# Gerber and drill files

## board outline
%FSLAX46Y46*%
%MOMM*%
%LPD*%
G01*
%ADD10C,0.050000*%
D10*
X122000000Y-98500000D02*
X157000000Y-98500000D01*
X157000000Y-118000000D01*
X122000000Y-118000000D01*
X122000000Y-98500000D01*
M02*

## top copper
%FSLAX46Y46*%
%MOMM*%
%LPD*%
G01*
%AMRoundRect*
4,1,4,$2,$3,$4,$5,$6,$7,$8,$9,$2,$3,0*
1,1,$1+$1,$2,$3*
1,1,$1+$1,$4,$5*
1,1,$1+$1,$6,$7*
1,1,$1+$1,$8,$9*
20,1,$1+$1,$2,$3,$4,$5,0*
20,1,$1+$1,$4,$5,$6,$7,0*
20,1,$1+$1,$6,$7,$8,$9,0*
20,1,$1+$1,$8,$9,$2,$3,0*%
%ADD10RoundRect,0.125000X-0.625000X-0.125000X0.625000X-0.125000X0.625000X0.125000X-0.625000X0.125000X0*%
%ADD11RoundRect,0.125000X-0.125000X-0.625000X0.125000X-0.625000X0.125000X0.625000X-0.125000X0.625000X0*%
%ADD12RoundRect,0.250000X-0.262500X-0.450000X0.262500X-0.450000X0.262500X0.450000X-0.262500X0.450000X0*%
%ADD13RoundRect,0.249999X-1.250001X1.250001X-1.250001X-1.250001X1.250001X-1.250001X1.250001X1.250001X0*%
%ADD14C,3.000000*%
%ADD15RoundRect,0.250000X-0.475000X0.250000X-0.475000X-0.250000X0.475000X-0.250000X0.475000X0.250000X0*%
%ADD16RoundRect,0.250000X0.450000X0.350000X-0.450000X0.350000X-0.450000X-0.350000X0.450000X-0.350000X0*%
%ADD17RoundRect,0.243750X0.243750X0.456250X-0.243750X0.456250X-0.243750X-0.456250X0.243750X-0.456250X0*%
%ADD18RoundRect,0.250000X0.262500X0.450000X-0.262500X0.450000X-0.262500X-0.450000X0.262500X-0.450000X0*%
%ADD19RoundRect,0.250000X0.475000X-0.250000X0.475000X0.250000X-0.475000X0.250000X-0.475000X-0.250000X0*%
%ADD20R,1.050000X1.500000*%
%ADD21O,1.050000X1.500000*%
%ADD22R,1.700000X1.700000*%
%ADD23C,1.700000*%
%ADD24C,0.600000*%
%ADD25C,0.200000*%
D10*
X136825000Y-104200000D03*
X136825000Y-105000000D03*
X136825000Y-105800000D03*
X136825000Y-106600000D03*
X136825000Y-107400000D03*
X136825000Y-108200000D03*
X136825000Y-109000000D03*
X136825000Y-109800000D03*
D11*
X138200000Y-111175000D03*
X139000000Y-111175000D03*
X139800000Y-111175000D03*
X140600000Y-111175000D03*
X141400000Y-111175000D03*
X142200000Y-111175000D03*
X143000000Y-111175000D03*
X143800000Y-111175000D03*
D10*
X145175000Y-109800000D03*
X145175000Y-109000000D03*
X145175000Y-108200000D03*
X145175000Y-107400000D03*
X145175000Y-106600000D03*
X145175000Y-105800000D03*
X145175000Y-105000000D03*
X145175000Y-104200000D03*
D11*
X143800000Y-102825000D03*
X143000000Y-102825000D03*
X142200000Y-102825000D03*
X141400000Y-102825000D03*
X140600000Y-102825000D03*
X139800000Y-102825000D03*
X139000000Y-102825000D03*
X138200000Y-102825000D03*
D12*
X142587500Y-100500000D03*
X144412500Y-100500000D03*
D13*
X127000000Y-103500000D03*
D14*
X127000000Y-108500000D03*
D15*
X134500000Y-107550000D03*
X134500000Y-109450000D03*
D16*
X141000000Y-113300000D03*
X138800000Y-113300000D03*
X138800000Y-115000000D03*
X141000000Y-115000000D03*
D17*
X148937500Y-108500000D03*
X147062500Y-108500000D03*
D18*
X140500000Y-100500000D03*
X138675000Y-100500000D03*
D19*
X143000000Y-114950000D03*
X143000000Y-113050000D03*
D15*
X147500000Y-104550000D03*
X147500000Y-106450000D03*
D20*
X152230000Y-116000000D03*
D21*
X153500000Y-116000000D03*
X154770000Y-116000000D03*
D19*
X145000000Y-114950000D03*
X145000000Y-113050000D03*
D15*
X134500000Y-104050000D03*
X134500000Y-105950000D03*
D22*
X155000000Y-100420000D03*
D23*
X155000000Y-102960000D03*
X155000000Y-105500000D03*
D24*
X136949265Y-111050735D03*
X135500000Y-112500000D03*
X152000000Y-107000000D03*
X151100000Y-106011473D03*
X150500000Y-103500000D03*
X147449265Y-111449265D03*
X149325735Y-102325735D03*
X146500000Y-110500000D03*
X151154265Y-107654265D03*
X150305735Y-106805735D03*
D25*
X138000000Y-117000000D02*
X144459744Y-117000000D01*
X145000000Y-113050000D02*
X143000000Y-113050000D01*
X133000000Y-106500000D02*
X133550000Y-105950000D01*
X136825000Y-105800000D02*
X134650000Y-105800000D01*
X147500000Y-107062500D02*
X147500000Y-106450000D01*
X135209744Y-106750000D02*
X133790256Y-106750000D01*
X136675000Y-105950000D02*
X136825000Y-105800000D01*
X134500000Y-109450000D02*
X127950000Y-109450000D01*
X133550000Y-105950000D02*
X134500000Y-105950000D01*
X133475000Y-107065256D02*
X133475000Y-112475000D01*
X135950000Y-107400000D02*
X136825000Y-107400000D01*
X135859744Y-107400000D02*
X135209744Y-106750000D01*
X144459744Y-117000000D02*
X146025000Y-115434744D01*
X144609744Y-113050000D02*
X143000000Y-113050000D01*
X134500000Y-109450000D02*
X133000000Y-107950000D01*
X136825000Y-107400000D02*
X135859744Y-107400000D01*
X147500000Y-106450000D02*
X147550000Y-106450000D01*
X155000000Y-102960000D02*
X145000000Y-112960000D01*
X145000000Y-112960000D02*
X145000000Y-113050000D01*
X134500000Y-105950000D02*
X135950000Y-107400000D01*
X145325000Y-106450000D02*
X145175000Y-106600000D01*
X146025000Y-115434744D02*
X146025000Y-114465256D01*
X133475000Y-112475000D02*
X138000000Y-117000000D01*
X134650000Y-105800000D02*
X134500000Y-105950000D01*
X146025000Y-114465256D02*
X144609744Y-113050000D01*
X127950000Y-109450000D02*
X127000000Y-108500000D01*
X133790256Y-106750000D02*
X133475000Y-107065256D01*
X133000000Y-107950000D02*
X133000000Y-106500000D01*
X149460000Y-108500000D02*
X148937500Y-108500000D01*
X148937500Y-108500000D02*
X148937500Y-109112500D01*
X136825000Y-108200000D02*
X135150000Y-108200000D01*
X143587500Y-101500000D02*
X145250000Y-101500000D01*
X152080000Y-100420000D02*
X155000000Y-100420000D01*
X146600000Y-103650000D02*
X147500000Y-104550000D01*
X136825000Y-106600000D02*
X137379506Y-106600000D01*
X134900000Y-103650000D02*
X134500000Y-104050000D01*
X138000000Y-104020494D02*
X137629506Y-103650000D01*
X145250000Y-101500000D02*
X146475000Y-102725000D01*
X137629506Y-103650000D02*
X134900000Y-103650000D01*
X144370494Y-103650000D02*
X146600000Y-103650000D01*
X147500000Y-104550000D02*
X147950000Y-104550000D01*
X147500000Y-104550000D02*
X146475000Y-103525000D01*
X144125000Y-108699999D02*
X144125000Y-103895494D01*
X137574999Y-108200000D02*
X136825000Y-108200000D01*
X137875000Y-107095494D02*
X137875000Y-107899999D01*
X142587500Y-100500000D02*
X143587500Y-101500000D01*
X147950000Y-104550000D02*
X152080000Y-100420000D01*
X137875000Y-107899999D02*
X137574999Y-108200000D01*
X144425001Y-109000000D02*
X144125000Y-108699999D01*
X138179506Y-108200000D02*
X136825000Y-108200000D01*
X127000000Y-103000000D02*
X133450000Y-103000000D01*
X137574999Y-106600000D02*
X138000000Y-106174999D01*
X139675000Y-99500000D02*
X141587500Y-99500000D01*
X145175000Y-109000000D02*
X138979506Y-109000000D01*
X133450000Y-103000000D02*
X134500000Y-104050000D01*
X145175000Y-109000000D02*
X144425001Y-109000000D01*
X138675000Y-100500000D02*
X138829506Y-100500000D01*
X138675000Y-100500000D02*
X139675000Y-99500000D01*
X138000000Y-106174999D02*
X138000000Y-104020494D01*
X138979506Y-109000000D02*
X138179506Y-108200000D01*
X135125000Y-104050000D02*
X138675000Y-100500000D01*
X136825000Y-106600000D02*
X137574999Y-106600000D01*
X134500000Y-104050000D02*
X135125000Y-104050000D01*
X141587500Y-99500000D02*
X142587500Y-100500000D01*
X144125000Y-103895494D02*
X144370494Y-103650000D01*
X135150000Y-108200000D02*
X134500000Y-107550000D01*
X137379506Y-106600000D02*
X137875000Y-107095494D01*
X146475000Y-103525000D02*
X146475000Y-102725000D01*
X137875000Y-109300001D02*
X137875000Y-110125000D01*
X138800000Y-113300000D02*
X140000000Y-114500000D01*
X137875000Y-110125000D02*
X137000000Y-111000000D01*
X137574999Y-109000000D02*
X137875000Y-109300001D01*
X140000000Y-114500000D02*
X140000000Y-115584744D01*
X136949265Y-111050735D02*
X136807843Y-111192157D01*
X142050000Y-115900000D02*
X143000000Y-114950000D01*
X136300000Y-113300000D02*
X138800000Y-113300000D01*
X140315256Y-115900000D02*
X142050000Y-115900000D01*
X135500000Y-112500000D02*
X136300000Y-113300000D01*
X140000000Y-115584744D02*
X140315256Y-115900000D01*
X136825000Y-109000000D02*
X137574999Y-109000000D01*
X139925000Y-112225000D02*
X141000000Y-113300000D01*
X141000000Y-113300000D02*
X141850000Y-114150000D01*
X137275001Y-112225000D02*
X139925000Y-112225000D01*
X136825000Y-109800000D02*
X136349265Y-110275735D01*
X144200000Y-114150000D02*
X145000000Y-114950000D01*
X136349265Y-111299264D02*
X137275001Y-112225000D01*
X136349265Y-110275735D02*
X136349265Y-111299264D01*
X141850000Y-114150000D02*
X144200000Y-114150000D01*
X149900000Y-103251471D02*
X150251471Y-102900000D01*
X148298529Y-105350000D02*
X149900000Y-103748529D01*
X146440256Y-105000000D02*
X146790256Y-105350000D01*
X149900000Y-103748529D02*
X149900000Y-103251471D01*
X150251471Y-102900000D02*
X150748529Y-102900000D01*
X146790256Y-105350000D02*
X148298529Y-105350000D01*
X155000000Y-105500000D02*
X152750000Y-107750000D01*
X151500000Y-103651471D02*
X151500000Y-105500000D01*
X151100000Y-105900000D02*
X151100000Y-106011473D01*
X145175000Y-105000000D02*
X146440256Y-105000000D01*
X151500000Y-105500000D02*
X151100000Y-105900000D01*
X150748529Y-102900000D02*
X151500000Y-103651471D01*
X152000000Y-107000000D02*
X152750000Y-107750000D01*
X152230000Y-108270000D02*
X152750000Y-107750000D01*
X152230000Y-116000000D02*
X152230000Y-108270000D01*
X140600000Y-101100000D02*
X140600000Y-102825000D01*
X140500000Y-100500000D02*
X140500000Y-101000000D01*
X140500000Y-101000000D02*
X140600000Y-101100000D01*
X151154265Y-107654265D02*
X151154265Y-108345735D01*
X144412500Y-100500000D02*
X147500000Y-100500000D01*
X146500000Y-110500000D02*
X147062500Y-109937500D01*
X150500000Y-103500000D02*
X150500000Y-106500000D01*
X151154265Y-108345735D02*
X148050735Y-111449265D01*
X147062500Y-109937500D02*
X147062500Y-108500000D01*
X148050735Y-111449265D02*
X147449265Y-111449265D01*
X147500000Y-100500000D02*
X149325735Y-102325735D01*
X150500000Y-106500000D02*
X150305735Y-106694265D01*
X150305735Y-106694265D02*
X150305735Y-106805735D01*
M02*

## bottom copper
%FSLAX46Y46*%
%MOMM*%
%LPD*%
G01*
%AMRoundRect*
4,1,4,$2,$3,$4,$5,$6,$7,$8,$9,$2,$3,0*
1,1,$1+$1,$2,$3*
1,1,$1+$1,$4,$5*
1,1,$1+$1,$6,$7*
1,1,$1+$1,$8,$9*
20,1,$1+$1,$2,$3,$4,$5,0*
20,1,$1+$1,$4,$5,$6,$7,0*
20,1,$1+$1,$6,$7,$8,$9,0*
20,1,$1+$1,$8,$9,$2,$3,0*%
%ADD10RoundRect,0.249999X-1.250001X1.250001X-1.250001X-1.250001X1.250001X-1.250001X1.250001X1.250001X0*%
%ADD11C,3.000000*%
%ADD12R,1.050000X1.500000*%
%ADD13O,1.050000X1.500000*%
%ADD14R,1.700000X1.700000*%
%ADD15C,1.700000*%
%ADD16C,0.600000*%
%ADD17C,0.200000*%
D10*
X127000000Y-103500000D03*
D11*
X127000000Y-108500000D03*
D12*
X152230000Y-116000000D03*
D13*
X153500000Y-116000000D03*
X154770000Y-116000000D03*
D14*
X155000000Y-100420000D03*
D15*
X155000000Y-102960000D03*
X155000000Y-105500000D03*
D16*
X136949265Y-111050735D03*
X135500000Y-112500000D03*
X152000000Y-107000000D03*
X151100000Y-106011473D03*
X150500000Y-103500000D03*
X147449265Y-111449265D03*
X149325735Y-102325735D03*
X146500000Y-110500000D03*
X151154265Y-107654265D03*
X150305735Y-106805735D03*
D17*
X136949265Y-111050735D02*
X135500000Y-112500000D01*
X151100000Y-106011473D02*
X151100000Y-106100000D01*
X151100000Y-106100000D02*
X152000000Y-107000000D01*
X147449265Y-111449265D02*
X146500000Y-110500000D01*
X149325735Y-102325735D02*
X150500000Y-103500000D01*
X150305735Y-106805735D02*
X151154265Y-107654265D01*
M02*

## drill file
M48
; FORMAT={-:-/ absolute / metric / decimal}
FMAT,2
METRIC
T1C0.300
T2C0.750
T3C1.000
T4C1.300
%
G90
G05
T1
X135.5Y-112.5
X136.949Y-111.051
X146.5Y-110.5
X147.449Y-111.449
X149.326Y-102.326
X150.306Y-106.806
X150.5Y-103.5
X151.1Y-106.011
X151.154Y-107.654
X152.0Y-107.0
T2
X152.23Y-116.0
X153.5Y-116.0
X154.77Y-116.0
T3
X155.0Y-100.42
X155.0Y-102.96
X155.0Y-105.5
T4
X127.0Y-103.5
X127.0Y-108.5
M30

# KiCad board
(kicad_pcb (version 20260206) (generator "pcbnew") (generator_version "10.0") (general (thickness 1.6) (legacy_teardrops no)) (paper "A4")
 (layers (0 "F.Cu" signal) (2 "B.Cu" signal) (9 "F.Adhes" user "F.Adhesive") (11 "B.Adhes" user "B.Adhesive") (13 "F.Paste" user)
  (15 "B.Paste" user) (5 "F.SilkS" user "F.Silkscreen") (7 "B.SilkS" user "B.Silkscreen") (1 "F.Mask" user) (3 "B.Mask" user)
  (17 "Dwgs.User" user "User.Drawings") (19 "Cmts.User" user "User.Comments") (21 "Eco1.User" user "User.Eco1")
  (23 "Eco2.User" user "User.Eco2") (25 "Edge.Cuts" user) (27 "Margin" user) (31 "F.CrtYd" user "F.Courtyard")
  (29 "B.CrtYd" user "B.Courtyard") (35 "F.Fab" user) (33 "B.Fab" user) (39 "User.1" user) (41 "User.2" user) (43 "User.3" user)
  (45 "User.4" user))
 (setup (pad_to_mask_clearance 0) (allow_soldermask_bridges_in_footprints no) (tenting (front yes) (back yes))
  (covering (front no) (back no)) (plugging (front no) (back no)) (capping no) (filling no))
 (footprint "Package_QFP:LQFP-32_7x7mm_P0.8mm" (layer "F.Cu") (at 141 107)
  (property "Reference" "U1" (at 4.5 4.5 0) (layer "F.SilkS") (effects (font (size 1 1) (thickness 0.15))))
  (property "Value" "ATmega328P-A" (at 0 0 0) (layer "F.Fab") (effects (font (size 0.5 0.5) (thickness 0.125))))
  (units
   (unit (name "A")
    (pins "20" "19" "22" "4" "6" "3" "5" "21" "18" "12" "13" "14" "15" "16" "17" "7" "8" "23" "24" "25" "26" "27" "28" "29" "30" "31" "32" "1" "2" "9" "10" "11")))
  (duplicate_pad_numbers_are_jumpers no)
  (pad "1" smd roundrect (at -4.175 -2.8) (size 1.5 0.5) (layers "F.Cu" "F.Mask" "F.Paste") (roundrect_rratio 0.25)
   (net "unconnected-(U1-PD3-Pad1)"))
  (pad "2" smd roundrect (at -4.175 -2) (size 1.5 0.5) (layers "F.Cu" "F.Mask" "F.Paste") (roundrect_rratio 0.25)
   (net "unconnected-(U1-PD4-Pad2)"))
  (pad "3" smd roundrect (at -4.175 -1.2) (size 1.5 0.5) (layers "F.Cu" "F.Mask" "F.Paste") (roundrect_rratio 0.25) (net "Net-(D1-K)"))
  (pad "4" smd roundrect (at -4.175 -0.4) (size 1.5 0.5) (layers "F.Cu" "F.Mask" "F.Paste") (roundrect_rratio 0.25) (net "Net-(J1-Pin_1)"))
  (pad "5" smd roundrect (at -4.175 0.4) (size 1.5 0.5) (layers "F.Cu" "F.Mask" "F.Paste") (roundrect_rratio 0.25) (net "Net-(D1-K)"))
  (pad "6" smd roundrect (at -4.175 1.2) (size 1.5 0.5) (layers "F.Cu" "F.Mask" "F.Paste") (roundrect_rratio 0.25) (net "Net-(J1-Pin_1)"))
  (pad "7" smd roundrect (at -4.175 2) (size 1.5 0.5) (layers "F.Cu" "F.Mask" "F.Paste") (roundrect_rratio 0.25)
   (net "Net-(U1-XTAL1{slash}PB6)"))
  (pad "8" smd roundrect (at -4.175 2.8) (size 1.5 0.5) (layers "F.Cu" "F.Mask" "F.Paste") (roundrect_rratio 0.25)
   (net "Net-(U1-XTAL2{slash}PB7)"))
  (pad "9" smd roundrect (at -2.8 4.175) (size 0.5 1.5) (layers "F.Cu" "F.Mask" "F.Paste") (roundrect_rratio 0.25)
   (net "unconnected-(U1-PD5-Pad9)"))
  (pad "10" smd roundrect (at -2 4.175) (size 0.5 1.5) (layers "F.Cu" "F.Mask" "F.Paste") (roundrect_rratio 0.25)
   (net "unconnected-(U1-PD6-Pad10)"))
  (pad "11" smd roundrect (at -1.2 4.175) (size 0.5 1.5) (layers "F.Cu" "F.Mask" "F.Paste") (roundrect_rratio 0.25)
   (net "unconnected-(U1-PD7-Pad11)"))
  (pad "12" smd roundrect (at -0.4 4.175) (size 0.5 1.5) (layers "F.Cu" "F.Mask" "F.Paste") (roundrect_rratio 0.25)
   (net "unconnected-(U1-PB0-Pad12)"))
  (pad "13" smd roundrect (at 0.4 4.175) (size 0.5 1.5) (layers "F.Cu" "F.Mask" "F.Paste") (roundrect_rratio 0.25)
   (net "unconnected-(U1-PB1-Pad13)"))
  (pad "14" smd roundrect (at 1.2 4.175) (size 0.5 1.5) (layers "F.Cu" "F.Mask" "F.Paste") (roundrect_rratio 0.25)
   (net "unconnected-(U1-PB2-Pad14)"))
  (pad "15" smd roundrect (at 2 4.175) (size 0.5 1.5) (layers "F.Cu" "F.Mask" "F.Paste") (roundrect_rratio 0.25)
   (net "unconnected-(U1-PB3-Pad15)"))
  (pad "16" smd roundrect (at 2.8 4.175) (size 0.5 1.5) (layers "F.Cu" "F.Mask" "F.Paste") (roundrect_rratio 0.25)
   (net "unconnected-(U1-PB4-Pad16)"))
  (pad "17" smd roundrect (at 4.175 2.8) (size 1.5 0.5) (layers "F.Cu" "F.Mask" "F.Paste") (roundrect_rratio 0.25)
   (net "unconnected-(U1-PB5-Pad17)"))
  (pad "18" smd roundrect (at 4.175 2) (size 1.5 0.5) (layers "F.Cu" "F.Mask" "F.Paste") (roundrect_rratio 0.25) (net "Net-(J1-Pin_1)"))
  (pad "19" smd roundrect (at 4.175 1.2) (size 1.5 0.5) (layers "F.Cu" "F.Mask" "F.Paste") (roundrect_rratio 0.25)
   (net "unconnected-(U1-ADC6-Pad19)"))
  (pad "20" smd roundrect (at 4.175 0.4) (size 1.5 0.5) (layers "F.Cu" "F.Mask" "F.Paste") (roundrect_rratio 0.25)
   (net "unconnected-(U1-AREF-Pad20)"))
  (pad "21" smd roundrect (at 4.175 -0.4) (size 1.5 0.5) (layers "F.Cu" "F.Mask" "F.Paste") (roundrect_rratio 0.25) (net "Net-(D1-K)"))
  (pad "22" smd roundrect (at 4.175 -1.2) (size 1.5 0.5) (layers "F.Cu" "F.Mask" "F.Paste") (roundrect_rratio 0.25)
   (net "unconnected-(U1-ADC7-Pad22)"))
  (pad "23" smd roundrect (at 4.175 -2) (size 1.5 0.5) (layers "F.Cu" "F.Mask" "F.Paste") (roundrect_rratio 0.25) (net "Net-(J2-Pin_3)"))
  (pad "24" smd roundrect (at 4.175 -2.8) (size 1.5 0.5) (layers "F.Cu" "F.Mask" "F.Paste") (roundrect_rratio 0.25)
   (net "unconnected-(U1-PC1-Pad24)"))
  (pad "25" smd roundrect (at 2.8 -4.175) (size 0.5 1.5) (layers "F.Cu" "F.Mask" "F.Paste") (roundrect_rratio 0.25)
   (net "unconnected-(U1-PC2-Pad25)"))
  (pad "26" smd roundrect (at 2 -4.175) (size 0.5 1.5) (layers "F.Cu" "F.Mask" "F.Paste") (roundrect_rratio 0.25)
   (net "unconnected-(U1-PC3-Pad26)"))
  (pad "27" smd roundrect (at 1.2 -4.175) (size 0.5 1.5) (layers "F.Cu" "F.Mask" "F.Paste") (roundrect_rratio 0.25)
   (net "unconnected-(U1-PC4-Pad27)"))
  (pad "28" smd roundrect (at 0.4 -4.175) (size 0.5 1.5) (layers "F.Cu" "F.Mask" "F.Paste") (roundrect_rratio 0.25)
   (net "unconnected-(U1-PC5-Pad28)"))
  (pad "29" smd roundrect (at -0.4 -4.175) (size 0.5 1.5) (layers "F.Cu" "F.Mask" "F.Paste") (roundrect_rratio 0.25)
   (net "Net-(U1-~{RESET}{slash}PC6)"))
  (pad "30" smd roundrect (at -1.2 -4.175) (size 0.5 1.5) (layers "F.Cu" "F.Mask" "F.Paste") (roundrect_rratio 0.25)
   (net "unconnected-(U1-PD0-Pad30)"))
  (pad "31" smd roundrect (at -2 -4.175) (size 0.5 1.5) (layers "F.Cu" "F.Mask" "F.Paste") (roundrect_rratio 0.25)
   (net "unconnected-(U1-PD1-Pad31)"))
  (pad "32" smd roundrect (at -2.8 -4.175) (size 0.5 1.5) (layers "F.Cu" "F.Mask" "F.Paste") (roundrect_rratio 0.25)
   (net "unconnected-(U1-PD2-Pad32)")))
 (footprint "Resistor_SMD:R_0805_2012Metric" (layer "F.Cu") (at 143.5 100.5)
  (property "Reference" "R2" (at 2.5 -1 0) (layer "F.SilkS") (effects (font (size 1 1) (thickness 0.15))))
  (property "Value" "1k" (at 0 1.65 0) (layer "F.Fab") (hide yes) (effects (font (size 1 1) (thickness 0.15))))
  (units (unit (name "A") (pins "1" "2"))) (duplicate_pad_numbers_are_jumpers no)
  (pad "1" smd roundrect (at -0.9125 0) (size 1.025 1.4) (layers "F.Cu" "F.Mask" "F.Paste") (roundrect_rratio 0.243902)
   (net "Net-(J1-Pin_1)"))
  (pad "2" smd roundrect (at 0.9125 0) (size 1.025 1.4) (layers "F.Cu" "F.Mask" "F.Paste") (roundrect_rratio 0.243902) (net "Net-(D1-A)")))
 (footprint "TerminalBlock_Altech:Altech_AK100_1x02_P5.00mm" (layer "F.Cu") (at 127 103.5 -90)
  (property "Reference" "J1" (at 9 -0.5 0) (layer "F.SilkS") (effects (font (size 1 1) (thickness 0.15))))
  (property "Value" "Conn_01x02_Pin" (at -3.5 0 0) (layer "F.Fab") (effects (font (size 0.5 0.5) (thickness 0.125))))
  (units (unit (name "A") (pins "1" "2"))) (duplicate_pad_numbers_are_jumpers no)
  (pad "1" thru_hole roundrect (at 0 0 270) (size 3 3) (drill 1.3) (layers "*.Cu" "*.Mask") (remove_unused_layers no)
   (roundrect_rratio 0.083333) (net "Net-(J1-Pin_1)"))
  (pad "2" thru_hole circle (at 5 0 270) (size 3 3) (drill 1.3) (layers "*.Cu" "*.Mask") (remove_unused_layers no) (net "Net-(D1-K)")))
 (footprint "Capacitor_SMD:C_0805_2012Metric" (layer "F.Cu") (at 134.5 108.5 -90)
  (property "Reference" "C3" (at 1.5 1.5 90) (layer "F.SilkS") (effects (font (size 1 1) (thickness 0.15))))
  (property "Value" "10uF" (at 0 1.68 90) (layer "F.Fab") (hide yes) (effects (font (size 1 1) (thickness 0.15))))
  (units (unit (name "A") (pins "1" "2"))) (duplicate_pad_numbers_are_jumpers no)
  (pad "1" smd roundrect (at -0.95 0 270) (size 1 1.45) (layers "F.Cu" "F.Mask" "F.Paste") (roundrect_rratio 0.25) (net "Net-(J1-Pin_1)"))
  (pad "2" smd roundrect (at 0.95 0 270) (size 1 1.45) (layers "F.Cu" "F.Mask" "F.Paste") (roundrect_rratio 0.25) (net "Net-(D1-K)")))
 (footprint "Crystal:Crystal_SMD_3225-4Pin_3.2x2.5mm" (layer "F.Cu") (at 139.9 114.15 180)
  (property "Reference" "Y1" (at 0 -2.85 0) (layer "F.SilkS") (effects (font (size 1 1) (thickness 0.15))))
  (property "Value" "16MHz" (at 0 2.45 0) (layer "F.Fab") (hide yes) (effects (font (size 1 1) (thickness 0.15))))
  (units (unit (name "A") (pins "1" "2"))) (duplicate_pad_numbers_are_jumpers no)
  (pad "1" smd roundrect (at -1.1 0.85 180) (size 1.4 1.2) (layers "F.Cu" "F.Mask" "F.Paste") (roundrect_rratio 0.208333)
   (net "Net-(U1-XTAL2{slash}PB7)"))
  (pad "2" smd roundrect (at 1.1 0.85 180) (size 1.4 1.2) (layers "F.Cu" "F.Mask" "F.Paste") (roundrect_rratio 0.208333)
   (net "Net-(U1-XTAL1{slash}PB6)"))
  (pad "3" smd roundrect (at 1.1 -0.85 180) (size 1.4 1.2) (layers "F.Cu" "F.Mask" "F.Paste") (roundrect_rratio 0.208333))
  (pad "4" smd roundrect (at -1.1 -0.85 180) (size 1.4 1.2) (layers "F.Cu" "F.Mask" "F.Paste") (roundrect_rratio 0.208333)))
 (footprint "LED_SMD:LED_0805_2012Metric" (layer "F.Cu") (at 148 108.5 180)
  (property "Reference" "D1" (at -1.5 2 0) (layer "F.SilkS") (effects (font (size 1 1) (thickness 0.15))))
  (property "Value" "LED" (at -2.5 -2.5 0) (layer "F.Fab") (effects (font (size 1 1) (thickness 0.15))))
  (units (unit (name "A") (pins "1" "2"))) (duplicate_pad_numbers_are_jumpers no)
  (pad "1" smd roundrect (at -0.9375 0 180) (size 0.975 1.4) (layers "F.Cu" "F.Mask" "F.Paste") (roundrect_rratio 0.25) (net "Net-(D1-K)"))
  (pad "2" smd roundrect (at 0.9375 0 180) (size 0.975 1.4) (layers "F.Cu" "F.Mask" "F.Paste") (roundrect_rratio 0.25) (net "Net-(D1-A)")))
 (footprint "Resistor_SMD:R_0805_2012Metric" (layer "F.Cu") (at 139.5875 100.5 180)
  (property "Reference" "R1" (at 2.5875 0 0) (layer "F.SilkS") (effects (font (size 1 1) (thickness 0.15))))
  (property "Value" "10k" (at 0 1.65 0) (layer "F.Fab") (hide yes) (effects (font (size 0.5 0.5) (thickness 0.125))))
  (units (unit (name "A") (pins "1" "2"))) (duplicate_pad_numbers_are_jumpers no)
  (pad "1" smd roundrect (at -0.9125 0 180) (size 1.025 1.4) (layers "F.Cu" "F.Mask" "F.Paste") (roundrect_rratio 0.243902)
   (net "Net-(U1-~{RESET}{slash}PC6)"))
  (pad "2" smd roundrect (at 0.9125 0 180) (size 1.025 1.4) (layers "F.Cu" "F.Mask" "F.Paste") (roundrect_rratio 0.243902)
   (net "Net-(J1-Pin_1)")))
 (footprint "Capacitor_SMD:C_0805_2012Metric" (layer "F.Cu") (at 143 114 90)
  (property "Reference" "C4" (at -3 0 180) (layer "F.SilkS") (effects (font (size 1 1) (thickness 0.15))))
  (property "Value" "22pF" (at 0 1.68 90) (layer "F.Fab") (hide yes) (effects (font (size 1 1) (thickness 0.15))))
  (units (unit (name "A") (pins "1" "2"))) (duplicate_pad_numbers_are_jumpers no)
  (pad "1" smd roundrect (at -0.95 0 90) (size 1 1.45) (layers "F.Cu" "F.Mask" "F.Paste") (roundrect_rratio 0.25)
   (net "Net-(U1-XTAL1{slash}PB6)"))
  (pad "2" smd roundrect (at 0.95 0 90) (size 1 1.45) (layers "F.Cu" "F.Mask" "F.Paste") (roundrect_rratio 0.25) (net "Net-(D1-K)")))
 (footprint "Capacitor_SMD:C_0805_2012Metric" (layer "F.Cu") (at 147.5 105.5 -90)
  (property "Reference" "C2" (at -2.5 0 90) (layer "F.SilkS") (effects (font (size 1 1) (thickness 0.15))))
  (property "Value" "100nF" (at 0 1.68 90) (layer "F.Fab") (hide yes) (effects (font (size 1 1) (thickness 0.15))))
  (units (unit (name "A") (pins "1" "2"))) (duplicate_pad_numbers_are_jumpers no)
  (pad "1" smd roundrect (at -0.95 0 270) (size 1 1.45) (layers "F.Cu" "F.Mask" "F.Paste") (roundrect_rratio 0.25) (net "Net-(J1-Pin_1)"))
  (pad "2" smd roundrect (at 0.95 0 270) (size 1 1.45) (layers "F.Cu" "F.Mask" "F.Paste") (roundrect_rratio 0.25) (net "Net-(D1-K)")))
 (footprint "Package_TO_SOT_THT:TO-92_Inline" (layer "F.Cu") (at 152.23 116)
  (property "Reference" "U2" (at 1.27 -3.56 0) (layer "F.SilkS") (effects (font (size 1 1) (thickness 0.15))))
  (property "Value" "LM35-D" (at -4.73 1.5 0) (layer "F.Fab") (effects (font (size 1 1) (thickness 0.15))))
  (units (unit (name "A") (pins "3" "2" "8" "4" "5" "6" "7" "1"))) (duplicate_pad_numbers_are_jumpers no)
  (pad "1" thru_hole rect (at 0 0) (size 1.05 1.5) (drill 0.75) (layers "*.Cu" "*.Mask") (remove_unused_layers no) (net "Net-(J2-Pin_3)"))
  (pad "2" thru_hole oval (at 1.27 0) (size 1.05 1.5) (drill 0.75) (layers "*.Cu" "*.Mask") (remove_unused_layers no)
   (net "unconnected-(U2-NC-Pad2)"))
  (pad "3" thru_hole oval (at 2.54 0) (size 1.05 1.5) (drill 0.75) (layers "*.Cu" "*.Mask") (remove_unused_layers no)
   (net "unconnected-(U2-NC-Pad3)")))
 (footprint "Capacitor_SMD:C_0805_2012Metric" (layer "F.Cu") (at 145 114 90)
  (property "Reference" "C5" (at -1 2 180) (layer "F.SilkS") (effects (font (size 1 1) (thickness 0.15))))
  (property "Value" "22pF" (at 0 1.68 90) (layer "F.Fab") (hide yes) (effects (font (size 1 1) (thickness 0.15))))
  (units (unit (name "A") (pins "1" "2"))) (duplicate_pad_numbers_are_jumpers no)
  (pad "1" smd roundrect (at -0.95 0 90) (size 1 1.45) (layers "F.Cu" "F.Mask" "F.Paste") (roundrect_rratio 0.25)
   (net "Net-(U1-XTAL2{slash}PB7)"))
  (pad "2" smd roundrect (at 0.95 0 90) (size 1 1.45) (layers "F.Cu" "F.Mask" "F.Paste") (roundrect_rratio 0.25) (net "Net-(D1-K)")))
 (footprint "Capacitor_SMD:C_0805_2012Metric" (layer "F.Cu") (at 134.5 105 -90)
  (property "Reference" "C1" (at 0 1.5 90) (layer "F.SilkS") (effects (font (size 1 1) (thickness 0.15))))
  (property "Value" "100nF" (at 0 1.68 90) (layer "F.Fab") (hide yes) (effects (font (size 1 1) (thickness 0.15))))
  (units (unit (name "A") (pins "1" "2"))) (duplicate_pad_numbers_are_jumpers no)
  (pad "1" smd roundrect (at -0.95 0 270) (size 1 1.45) (layers "F.Cu" "F.Mask" "F.Paste") (roundrect_rratio 0.25) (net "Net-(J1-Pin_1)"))
  (pad "2" smd roundrect (at 0.95 0 270) (size 1 1.45) (layers "F.Cu" "F.Mask" "F.Paste") (roundrect_rratio 0.25) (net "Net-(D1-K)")))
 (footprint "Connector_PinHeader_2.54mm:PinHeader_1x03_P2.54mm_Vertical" (layer "F.Cu") (at 155 100.42)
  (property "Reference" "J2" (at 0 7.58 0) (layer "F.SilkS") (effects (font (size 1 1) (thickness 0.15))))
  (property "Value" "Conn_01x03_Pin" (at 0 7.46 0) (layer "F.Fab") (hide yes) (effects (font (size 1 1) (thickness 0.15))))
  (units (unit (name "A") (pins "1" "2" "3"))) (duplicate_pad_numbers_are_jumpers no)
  (pad "1" thru_hole rect (at 0 0) (size 1.7 1.7) (drill 1) (layers "*.Cu" "*.Mask") (remove_unused_layers no) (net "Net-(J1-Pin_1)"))
  (pad "2" thru_hole circle (at 0 2.54) (size 1.7 1.7) (drill 1) (layers "*.Cu" "*.Mask") (remove_unused_layers no) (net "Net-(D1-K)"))
  (pad "3" thru_hole circle (at 0 5.08) (size 1.7 1.7) (drill 1) (layers "*.Cu" "*.Mask") (remove_unused_layers no) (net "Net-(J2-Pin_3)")))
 (gr_rect (start 122 98.5) (end 157 118) (stroke (width 0.05) (type default)) (fill no) (layer "Edge.Cuts"))
 (segment (start 138 117) (end 144.459744 117) (width 0.2) (layer "F.Cu") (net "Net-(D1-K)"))
 (segment (start 145 113.05) (end 143 113.05) (width 0.2) (layer "F.Cu") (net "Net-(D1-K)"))
 (segment (start 133 106.5) (end 133.55 105.95) (width 0.2) (layer "F.Cu") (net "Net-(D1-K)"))
 (segment (start 136.825 105.8) (end 134.65 105.8) (width 0.2) (layer "F.Cu") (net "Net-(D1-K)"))
 (segment (start 147.5 107.0625) (end 147.5 106.45) (width 0.2) (layer "F.Cu") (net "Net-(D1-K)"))
 (segment (start 135.209744 106.75) (end 133.790256 106.75) (width 0.2) (layer "F.Cu") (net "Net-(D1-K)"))
 (segment (start 136.675 105.95) (end 136.825 105.8) (width 0.2) (layer "F.Cu") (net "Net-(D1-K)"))
 (segment (start 134.5 109.45) (end 127.95 109.45) (width 0.2) (layer "F.Cu") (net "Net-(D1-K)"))
 (segment (start 133.55 105.95) (end 134.5 105.95) (width 0.2) (layer "F.Cu") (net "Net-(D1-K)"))
 (segment (start 133.475 107.065256) (end 133.475 112.475) (width 0.2) (layer "F.Cu") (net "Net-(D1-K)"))
 (segment (start 135.95 107.4) (end 136.825 107.4) (width 0.2) (layer "F.Cu") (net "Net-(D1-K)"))
 (segment (start 135.859744 107.4) (end 135.209744 106.75) (width 0.2) (layer "F.Cu") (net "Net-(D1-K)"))
 (segment (start 144.459744 117) (end 146.025 115.434744) (width 0.2) (layer "F.Cu") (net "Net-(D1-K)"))
 (segment (start 144.609744 113.05) (end 143 113.05) (width 0.2) (layer "F.Cu") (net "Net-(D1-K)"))
 (segment (start 134.5 109.45) (end 133 107.95) (width 0.2) (layer "F.Cu") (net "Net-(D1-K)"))
 (segment (start 136.825 107.4) (end 135.859744 107.4) (width 0.2) (layer "F.Cu") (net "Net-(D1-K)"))
 (segment (start 147.5 106.45) (end 147.55 106.45) (width 0.2) (layer "F.Cu") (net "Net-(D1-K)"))
 (segment (start 155 102.96) (end 145 112.96) (width 0.2) (layer "F.Cu") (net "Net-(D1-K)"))
 (segment (start 145 112.96) (end 145 113.05) (width 0.2) (layer "F.Cu") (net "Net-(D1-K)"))
 (segment (start 134.5 105.95) (end 135.95 107.4) (width 0.2) (layer "F.Cu") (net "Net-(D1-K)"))
 (segment (start 145.325 106.45) (end 145.175 106.6) (width 0.2) (layer "F.Cu") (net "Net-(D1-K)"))
 (segment (start 146.025 115.434744) (end 146.025 114.465256) (width 0.2) (layer "F.Cu") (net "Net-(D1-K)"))
 (segment (start 133.475 112.475) (end 138 117) (width 0.2) (layer "F.Cu") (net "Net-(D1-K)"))
 (segment (start 134.65 105.8) (end 134.5 105.95) (width 0.2) (layer "F.Cu") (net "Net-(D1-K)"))
 (segment (start 146.025 114.465256) (end 144.609744 113.05) (width 0.2) (layer "F.Cu") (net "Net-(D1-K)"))
 (segment (start 127.95 109.45) (end 127 108.5) (width 0.2) (layer "F.Cu") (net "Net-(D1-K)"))
 (segment (start 133.790256 106.75) (end 133.475 107.065256) (width 0.2) (layer "F.Cu") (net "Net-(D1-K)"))
 (segment (start 133 107.95) (end 133 106.5) (width 0.2) (layer "F.Cu") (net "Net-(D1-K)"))
 (segment (start 149.46 108.5) (end 148.9375 108.5) (width 0.2) (layer "F.Cu") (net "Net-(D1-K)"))
 (segment (start 148.9375 108.5) (end 148.9375 109.1125) (width 0.2) (layer "F.Cu") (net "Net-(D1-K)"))
 (segment (start 136.825 108.2) (end 135.15 108.2) (width 0.2) (layer "F.Cu") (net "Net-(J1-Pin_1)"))
 (segment (start 143.5875 101.5) (end 145.25 101.5) (width 0.2) (layer "F.Cu") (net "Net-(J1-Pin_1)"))
 (segment (start 152.08 100.42) (end 155 100.42) (width 0.2) (layer "F.Cu") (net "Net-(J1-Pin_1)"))
 (segment (start 146.6 103.65) (end 147.5 104.55) (width 0.2) (layer "F.Cu") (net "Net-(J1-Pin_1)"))
 (segment (start 136.825 106.6) (end 137.379506 106.6) (width 0.2) (layer "F.Cu") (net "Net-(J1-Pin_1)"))
 (segment (start 134.9 103.65) (end 134.5 104.05) (width 0.2) (layer "F.Cu") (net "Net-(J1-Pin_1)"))
 (segment (start 138 104.020494) (end 137.629506 103.65) (width 0.2) (layer "F.Cu") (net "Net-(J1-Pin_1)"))
 (segment (start 145.25 101.5) (end 146.475 102.725) (width 0.2) (layer "F.Cu") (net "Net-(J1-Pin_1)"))
 (segment (start 137.629506 103.65) (end 134.9 103.65) (width 0.2) (layer "F.Cu") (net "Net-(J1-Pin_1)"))
 (segment (start 144.370494 103.65) (end 146.6 103.65) (width 0.2) (layer "F.Cu") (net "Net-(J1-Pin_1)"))
 (segment (start 147.5 104.55) (end 147.95 104.55) (width 0.2) (layer "F.Cu") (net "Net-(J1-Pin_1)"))
 (segment (start 147.5 104.55) (end 146.475 103.525) (width 0.2) (layer "F.Cu") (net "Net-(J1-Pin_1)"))
 (segment (start 144.125 108.699999) (end 144.125 103.895494) (width 0.2) (layer "F.Cu") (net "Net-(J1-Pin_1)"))
 (segment (start 137.574999 108.2) (end 136.825 108.2) (width 0.2) (layer "F.Cu") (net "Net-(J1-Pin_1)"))
 (segment (start 137.875 107.095494) (end 137.875 107.899999) (width 0.2) (layer "F.Cu") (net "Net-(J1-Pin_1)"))
 (segment (start 142.5875 100.5) (end 143.5875 101.5) (width 0.2) (layer "F.Cu") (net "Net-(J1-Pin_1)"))
 (segment (start 147.95 104.55) (end 152.08 100.42) (width 0.2) (layer "F.Cu") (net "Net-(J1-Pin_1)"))
 (segment (start 137.875 107.899999) (end 137.574999 108.2) (width 0.2) (layer "F.Cu") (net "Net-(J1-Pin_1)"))
 (segment (start 144.425001 109) (end 144.125 108.699999) (width 0.2) (layer "F.Cu") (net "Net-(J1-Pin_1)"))
 (segment (start 138.179506 108.2) (end 136.825 108.2) (width 0.2) (layer "F.Cu") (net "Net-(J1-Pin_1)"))
 (segment (start 127 103) (end 133.45 103) (width 0.2) (layer "F.Cu") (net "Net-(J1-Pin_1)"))
 (segment (start 137.574999 106.6) (end 138 106.174999) (width 0.2) (layer "F.Cu") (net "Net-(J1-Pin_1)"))
 (segment (start 139.675 99.5) (end 141.5875 99.5) (width 0.2) (layer "F.Cu") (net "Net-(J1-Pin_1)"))
 (segment (start 145.175 109) (end 138.979506 109) (width 0.2) (layer "F.Cu") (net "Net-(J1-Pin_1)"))
 (segment (start 133.45 103) (end 134.5 104.05) (width 0.2) (layer "F.Cu") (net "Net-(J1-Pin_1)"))
 (segment (start 145.175 109) (end 144.425001 109) (width 0.2) (layer "F.Cu") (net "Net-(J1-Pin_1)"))
 (segment (start 138.675 100.5) (end 138.829506 100.5) (width 0.2) (layer "F.Cu") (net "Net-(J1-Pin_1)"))
 (segment (start 138.675 100.5) (end 139.675 99.5) (width 0.2) (layer "F.Cu") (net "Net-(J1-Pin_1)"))
 (segment (start 138 106.174999) (end 138 104.020494) (width 0.2) (layer "F.Cu") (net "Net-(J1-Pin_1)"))
 (segment (start 138.979506 109) (end 138.179506 108.2) (width 0.2) (layer "F.Cu") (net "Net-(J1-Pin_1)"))
 (segment (start 135.125 104.05) (end 138.675 100.5) (width 0.2) (layer "F.Cu") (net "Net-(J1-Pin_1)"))
 (segment (start 136.825 106.6) (end 137.574999 106.6) (width 0.2) (layer "F.Cu") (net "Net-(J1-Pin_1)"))
 (segment (start 134.5 104.05) (end 135.125 104.05) (width 0.2) (layer "F.Cu") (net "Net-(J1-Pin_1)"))
 (segment (start 141.5875 99.5) (end 142.5875 100.5) (width 0.2) (layer "F.Cu") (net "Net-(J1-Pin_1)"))
 (segment (start 144.125 103.895494) (end 144.370494 103.65) (width 0.2) (layer "F.Cu") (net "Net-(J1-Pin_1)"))
 (segment (start 135.15 108.2) (end 134.5 107.55) (width 0.2) (layer "F.Cu") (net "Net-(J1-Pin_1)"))
 (segment (start 137.379506 106.6) (end 137.875 107.095494) (width 0.2) (layer "F.Cu") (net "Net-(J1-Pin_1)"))
 (segment (start 146.475 103.525) (end 146.475 102.725) (width 0.2) (layer "F.Cu") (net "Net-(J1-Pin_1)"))
 (segment (start 137.875 109.300001) (end 137.875 110.125) (width 0.2) (layer "F.Cu") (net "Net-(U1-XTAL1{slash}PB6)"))
 (segment (start 138.8 113.3) (end 140 114.5) (width 0.2) (layer "F.Cu") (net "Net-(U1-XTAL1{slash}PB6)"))
 (segment (start 137.875 110.125) (end 137 111) (width 0.2) (layer "F.Cu") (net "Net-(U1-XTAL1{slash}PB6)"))
 (segment (start 137.574999 109) (end 137.875 109.300001) (width 0.2) (layer "F.Cu") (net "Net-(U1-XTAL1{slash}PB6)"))
 (segment (start 140 114.5) (end 140 115.584744) (width 0.2) (layer "F.Cu") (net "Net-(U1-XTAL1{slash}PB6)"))
 (segment (start 136.949265 111.050735) (end 136.807843 111.192157) (width 0.2) (layer "F.Cu") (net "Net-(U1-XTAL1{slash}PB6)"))
 (segment (start 142.05 115.9) (end 143 114.95) (width 0.2) (layer "F.Cu") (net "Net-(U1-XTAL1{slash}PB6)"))
 (segment (start 136.3 113.3) (end 138.8 113.3) (width 0.2) (layer "F.Cu") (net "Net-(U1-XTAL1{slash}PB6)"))
 (segment (start 140.315256 115.9) (end 142.05 115.9) (width 0.2) (layer "F.Cu") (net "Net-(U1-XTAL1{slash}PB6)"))
 (segment (start 135.5 112.5) (end 136.3 113.3) (width 0.2) (layer "F.Cu") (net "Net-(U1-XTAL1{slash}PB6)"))
 (segment (start 140 115.584744) (end 140.315256 115.9) (width 0.2) (layer "F.Cu") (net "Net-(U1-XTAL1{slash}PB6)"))
 (segment (start 136.825 109) (end 137.574999 109) (width 0.2) (layer "F.Cu") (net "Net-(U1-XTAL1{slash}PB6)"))
 (via (at 136.949265 111.050735) (size 0.6) (drill 0.3) (layers "F.Cu" "B.Cu") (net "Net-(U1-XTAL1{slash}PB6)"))
 (via (at 135.5 112.5) (size 0.6) (drill 0.3) (layers "F.Cu" "B.Cu") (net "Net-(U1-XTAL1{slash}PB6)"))
 (segment (start 136.949265 111.050735) (end 135.5 112.5) (width 0.2) (layer "B.Cu") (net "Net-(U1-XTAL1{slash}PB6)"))
 (segment (start 139.925 112.225) (end 141 113.3) (width 0.2) (layer "F.Cu") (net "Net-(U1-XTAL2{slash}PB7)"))
 (segment (start 141 113.3) (end 141.85 114.15) (width 0.2) (layer "F.Cu") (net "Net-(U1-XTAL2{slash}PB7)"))
 (segment (start 137.275001 112.225) (end 139.925 112.225) (width 0.2) (layer "F.Cu") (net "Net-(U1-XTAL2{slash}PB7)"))
 (segment (start 136.825 109.8) (end 136.349265 110.275735) (width 0.2) (layer "F.Cu") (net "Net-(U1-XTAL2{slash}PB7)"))
 (segment (start 144.2 114.15) (end 145 114.95) (width 0.2) (layer "F.Cu") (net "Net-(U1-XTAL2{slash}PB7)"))
 (segment (start 136.349265 111.299264) (end 137.275001 112.225) (width 0.2) (layer "F.Cu") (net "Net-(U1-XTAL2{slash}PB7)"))
 (segment (start 136.349265 110.275735) (end 136.349265 111.299264) (width 0.2) (layer "F.Cu") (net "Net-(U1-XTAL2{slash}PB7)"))
 (segment (start 141.85 114.15) (end 144.2 114.15) (width 0.2) (layer "F.Cu") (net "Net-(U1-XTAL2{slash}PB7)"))
 (segment (start 149.9 103.251471) (end 150.251471 102.9) (width 0.2) (layer "F.Cu") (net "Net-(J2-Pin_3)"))
 (segment (start 148.298529 105.35) (end 149.9 103.748529) (width 0.2) (layer "F.Cu") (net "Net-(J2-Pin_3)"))
 (segment (start 146.440256 105) (end 146.790256 105.35) (width 0.2) (layer "F.Cu") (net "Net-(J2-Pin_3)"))
 (segment (start 149.9 103.748529) (end 149.9 103.251471) (width 0.2) (layer "F.Cu") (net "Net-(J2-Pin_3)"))
 (segment (start 150.251471 102.9) (end 150.748529 102.9) (width 0.2) (layer "F.Cu") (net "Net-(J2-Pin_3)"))
 (segment (start 146.790256 105.35) (end 148.298529 105.35) (width 0.2) (layer "F.Cu") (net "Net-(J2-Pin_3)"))
 (segment (start 155 105.5) (end 152.75 107.75) (width 0.2) (layer "F.Cu") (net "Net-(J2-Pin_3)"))
 (segment (start 151.5 103.651471) (end 151.5 105.5) (width 0.2) (layer "F.Cu") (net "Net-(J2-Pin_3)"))
 (segment (start 151.1 105.9) (end 151.1 106.011473) (width 0.2) (layer "F.Cu") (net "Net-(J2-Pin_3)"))
 (segment (start 145.175 105) (end 146.440256 105) (width 0.2) (layer "F.Cu") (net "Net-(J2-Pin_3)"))
 (segment (start 151.5 105.5) (end 151.1 105.9) (width 0.2) (layer "F.Cu") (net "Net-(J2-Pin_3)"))
 (segment (start 150.748529 102.9) (end 151.5 103.651471) (width 0.2) (layer "F.Cu") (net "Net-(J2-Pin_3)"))
 (segment (start 152 107) (end 152.75 107.75) (width 0.2) (layer "F.Cu") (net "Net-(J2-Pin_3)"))
 (segment (start 152.23 108.27) (end 152.75 107.75) (width 0.2) (layer "F.Cu") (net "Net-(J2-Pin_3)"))
 (segment (start 152.23 116) (end 152.23 108.27) (width 0.2) (layer "F.Cu") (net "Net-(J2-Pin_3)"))
 (via (at 152 107) (size 0.6) (drill 0.3) (layers "F.Cu" "B.Cu") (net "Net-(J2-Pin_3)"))
 (via (at 151.1 106.011473) (size 0.6) (drill 0.3) (layers "F.Cu" "B.Cu") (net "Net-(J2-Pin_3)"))
 (segment (start 151.1 106.011473) (end 151.1 106.1) (width 0.2) (layer "B.Cu") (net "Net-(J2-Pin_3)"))
 (segment (start 151.1 106.1) (end 152 107) (width 0.2) (layer "B.Cu") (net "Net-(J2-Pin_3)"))
 (segment (start 140.6 101.1) (end 140.6 102.825) (width 0.2) (layer "F.Cu") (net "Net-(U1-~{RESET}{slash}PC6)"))
 (segment (start 140.5 100.5) (end 140.5 101) (width 0.2) (layer "F.Cu") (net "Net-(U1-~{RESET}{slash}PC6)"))
 (segment (start 140.5 101) (end 140.6 101.1) (width 0.2) (layer "F.Cu") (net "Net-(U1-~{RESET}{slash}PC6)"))
 (segment (start 151.154265 107.654265) (end 151.154265 108.345735) (width 0.2) (layer "F.Cu") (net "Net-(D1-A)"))
 (segment (start 144.4125 100.5) (end 147.5 100.5) (width 0.2) (layer "F.Cu") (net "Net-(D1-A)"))
 (segment (start 146.5 110.5) (end 147.0625 109.9375) (width 0.2) (layer "F.Cu") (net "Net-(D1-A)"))
 (segment (start 150.5 103.5) (end 150.5 106.5) (width 0.2) (layer "F.Cu") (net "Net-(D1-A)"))
 (segment (start 151.154265 108.345735) (end 148.050735 111.449265) (width 0.2) (layer "F.Cu") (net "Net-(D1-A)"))
 (segment (start 147.0625 109.9375) (end 147.0625 108.5) (width 0.2) (layer "F.Cu") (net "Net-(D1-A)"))
 (segment (start 148.050735 111.449265) (end 147.449265 111.449265) (width 0.2) (layer "F.Cu") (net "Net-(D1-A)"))
 (segment (start 147.5 100.5) (end 149.325735 102.325735) (width 0.2) (layer "F.Cu") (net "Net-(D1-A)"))
 (segment (start 150.5 106.5) (end 150.305735 106.694265) (width 0.2) (layer "F.Cu") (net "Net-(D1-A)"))
 (segment (start 150.305735 106.694265) (end 150.305735 106.805735) (width 0.2) (layer "F.Cu") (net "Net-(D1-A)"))
 (via (at 150.5 103.5) (size 0.6) (drill 0.3) (layers "F.Cu" "B.Cu") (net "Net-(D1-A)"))
 (via (at 147.449265 111.449265) (size 0.6) (drill 0.3) (layers "F.Cu" "B.Cu") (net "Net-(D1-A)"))
 (via (at 149.325735 102.325735) (size 0.6) (drill 0.3) (layers "F.Cu" "B.Cu") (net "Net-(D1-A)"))
 (via (at 146.5 110.5) (size 0.6) (drill 0.3) (layers "F.Cu" "B.Cu") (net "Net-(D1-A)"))
 (via (at 151.154265 107.654265) (size 0.6) (drill 0.3) (layers "F.Cu" "B.Cu") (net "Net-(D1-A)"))
 (via (at 150.305735 106.805735) (size 0.6) (drill 0.3) (layers "F.Cu" "B.Cu") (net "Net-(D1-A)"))
 (segment (start 147.449265 111.449265) (end 146.5 110.5) (width 0.2) (layer "B.Cu") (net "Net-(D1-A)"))
 (segment (start 149.325735 102.325735) (end 150.5 103.5) (width 0.2) (layer "B.Cu") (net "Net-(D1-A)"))
 (segment (start 150.305735 106.805735) (end 151.154265 107.654265) (width 0.2) (layer "B.Cu") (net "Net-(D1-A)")))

